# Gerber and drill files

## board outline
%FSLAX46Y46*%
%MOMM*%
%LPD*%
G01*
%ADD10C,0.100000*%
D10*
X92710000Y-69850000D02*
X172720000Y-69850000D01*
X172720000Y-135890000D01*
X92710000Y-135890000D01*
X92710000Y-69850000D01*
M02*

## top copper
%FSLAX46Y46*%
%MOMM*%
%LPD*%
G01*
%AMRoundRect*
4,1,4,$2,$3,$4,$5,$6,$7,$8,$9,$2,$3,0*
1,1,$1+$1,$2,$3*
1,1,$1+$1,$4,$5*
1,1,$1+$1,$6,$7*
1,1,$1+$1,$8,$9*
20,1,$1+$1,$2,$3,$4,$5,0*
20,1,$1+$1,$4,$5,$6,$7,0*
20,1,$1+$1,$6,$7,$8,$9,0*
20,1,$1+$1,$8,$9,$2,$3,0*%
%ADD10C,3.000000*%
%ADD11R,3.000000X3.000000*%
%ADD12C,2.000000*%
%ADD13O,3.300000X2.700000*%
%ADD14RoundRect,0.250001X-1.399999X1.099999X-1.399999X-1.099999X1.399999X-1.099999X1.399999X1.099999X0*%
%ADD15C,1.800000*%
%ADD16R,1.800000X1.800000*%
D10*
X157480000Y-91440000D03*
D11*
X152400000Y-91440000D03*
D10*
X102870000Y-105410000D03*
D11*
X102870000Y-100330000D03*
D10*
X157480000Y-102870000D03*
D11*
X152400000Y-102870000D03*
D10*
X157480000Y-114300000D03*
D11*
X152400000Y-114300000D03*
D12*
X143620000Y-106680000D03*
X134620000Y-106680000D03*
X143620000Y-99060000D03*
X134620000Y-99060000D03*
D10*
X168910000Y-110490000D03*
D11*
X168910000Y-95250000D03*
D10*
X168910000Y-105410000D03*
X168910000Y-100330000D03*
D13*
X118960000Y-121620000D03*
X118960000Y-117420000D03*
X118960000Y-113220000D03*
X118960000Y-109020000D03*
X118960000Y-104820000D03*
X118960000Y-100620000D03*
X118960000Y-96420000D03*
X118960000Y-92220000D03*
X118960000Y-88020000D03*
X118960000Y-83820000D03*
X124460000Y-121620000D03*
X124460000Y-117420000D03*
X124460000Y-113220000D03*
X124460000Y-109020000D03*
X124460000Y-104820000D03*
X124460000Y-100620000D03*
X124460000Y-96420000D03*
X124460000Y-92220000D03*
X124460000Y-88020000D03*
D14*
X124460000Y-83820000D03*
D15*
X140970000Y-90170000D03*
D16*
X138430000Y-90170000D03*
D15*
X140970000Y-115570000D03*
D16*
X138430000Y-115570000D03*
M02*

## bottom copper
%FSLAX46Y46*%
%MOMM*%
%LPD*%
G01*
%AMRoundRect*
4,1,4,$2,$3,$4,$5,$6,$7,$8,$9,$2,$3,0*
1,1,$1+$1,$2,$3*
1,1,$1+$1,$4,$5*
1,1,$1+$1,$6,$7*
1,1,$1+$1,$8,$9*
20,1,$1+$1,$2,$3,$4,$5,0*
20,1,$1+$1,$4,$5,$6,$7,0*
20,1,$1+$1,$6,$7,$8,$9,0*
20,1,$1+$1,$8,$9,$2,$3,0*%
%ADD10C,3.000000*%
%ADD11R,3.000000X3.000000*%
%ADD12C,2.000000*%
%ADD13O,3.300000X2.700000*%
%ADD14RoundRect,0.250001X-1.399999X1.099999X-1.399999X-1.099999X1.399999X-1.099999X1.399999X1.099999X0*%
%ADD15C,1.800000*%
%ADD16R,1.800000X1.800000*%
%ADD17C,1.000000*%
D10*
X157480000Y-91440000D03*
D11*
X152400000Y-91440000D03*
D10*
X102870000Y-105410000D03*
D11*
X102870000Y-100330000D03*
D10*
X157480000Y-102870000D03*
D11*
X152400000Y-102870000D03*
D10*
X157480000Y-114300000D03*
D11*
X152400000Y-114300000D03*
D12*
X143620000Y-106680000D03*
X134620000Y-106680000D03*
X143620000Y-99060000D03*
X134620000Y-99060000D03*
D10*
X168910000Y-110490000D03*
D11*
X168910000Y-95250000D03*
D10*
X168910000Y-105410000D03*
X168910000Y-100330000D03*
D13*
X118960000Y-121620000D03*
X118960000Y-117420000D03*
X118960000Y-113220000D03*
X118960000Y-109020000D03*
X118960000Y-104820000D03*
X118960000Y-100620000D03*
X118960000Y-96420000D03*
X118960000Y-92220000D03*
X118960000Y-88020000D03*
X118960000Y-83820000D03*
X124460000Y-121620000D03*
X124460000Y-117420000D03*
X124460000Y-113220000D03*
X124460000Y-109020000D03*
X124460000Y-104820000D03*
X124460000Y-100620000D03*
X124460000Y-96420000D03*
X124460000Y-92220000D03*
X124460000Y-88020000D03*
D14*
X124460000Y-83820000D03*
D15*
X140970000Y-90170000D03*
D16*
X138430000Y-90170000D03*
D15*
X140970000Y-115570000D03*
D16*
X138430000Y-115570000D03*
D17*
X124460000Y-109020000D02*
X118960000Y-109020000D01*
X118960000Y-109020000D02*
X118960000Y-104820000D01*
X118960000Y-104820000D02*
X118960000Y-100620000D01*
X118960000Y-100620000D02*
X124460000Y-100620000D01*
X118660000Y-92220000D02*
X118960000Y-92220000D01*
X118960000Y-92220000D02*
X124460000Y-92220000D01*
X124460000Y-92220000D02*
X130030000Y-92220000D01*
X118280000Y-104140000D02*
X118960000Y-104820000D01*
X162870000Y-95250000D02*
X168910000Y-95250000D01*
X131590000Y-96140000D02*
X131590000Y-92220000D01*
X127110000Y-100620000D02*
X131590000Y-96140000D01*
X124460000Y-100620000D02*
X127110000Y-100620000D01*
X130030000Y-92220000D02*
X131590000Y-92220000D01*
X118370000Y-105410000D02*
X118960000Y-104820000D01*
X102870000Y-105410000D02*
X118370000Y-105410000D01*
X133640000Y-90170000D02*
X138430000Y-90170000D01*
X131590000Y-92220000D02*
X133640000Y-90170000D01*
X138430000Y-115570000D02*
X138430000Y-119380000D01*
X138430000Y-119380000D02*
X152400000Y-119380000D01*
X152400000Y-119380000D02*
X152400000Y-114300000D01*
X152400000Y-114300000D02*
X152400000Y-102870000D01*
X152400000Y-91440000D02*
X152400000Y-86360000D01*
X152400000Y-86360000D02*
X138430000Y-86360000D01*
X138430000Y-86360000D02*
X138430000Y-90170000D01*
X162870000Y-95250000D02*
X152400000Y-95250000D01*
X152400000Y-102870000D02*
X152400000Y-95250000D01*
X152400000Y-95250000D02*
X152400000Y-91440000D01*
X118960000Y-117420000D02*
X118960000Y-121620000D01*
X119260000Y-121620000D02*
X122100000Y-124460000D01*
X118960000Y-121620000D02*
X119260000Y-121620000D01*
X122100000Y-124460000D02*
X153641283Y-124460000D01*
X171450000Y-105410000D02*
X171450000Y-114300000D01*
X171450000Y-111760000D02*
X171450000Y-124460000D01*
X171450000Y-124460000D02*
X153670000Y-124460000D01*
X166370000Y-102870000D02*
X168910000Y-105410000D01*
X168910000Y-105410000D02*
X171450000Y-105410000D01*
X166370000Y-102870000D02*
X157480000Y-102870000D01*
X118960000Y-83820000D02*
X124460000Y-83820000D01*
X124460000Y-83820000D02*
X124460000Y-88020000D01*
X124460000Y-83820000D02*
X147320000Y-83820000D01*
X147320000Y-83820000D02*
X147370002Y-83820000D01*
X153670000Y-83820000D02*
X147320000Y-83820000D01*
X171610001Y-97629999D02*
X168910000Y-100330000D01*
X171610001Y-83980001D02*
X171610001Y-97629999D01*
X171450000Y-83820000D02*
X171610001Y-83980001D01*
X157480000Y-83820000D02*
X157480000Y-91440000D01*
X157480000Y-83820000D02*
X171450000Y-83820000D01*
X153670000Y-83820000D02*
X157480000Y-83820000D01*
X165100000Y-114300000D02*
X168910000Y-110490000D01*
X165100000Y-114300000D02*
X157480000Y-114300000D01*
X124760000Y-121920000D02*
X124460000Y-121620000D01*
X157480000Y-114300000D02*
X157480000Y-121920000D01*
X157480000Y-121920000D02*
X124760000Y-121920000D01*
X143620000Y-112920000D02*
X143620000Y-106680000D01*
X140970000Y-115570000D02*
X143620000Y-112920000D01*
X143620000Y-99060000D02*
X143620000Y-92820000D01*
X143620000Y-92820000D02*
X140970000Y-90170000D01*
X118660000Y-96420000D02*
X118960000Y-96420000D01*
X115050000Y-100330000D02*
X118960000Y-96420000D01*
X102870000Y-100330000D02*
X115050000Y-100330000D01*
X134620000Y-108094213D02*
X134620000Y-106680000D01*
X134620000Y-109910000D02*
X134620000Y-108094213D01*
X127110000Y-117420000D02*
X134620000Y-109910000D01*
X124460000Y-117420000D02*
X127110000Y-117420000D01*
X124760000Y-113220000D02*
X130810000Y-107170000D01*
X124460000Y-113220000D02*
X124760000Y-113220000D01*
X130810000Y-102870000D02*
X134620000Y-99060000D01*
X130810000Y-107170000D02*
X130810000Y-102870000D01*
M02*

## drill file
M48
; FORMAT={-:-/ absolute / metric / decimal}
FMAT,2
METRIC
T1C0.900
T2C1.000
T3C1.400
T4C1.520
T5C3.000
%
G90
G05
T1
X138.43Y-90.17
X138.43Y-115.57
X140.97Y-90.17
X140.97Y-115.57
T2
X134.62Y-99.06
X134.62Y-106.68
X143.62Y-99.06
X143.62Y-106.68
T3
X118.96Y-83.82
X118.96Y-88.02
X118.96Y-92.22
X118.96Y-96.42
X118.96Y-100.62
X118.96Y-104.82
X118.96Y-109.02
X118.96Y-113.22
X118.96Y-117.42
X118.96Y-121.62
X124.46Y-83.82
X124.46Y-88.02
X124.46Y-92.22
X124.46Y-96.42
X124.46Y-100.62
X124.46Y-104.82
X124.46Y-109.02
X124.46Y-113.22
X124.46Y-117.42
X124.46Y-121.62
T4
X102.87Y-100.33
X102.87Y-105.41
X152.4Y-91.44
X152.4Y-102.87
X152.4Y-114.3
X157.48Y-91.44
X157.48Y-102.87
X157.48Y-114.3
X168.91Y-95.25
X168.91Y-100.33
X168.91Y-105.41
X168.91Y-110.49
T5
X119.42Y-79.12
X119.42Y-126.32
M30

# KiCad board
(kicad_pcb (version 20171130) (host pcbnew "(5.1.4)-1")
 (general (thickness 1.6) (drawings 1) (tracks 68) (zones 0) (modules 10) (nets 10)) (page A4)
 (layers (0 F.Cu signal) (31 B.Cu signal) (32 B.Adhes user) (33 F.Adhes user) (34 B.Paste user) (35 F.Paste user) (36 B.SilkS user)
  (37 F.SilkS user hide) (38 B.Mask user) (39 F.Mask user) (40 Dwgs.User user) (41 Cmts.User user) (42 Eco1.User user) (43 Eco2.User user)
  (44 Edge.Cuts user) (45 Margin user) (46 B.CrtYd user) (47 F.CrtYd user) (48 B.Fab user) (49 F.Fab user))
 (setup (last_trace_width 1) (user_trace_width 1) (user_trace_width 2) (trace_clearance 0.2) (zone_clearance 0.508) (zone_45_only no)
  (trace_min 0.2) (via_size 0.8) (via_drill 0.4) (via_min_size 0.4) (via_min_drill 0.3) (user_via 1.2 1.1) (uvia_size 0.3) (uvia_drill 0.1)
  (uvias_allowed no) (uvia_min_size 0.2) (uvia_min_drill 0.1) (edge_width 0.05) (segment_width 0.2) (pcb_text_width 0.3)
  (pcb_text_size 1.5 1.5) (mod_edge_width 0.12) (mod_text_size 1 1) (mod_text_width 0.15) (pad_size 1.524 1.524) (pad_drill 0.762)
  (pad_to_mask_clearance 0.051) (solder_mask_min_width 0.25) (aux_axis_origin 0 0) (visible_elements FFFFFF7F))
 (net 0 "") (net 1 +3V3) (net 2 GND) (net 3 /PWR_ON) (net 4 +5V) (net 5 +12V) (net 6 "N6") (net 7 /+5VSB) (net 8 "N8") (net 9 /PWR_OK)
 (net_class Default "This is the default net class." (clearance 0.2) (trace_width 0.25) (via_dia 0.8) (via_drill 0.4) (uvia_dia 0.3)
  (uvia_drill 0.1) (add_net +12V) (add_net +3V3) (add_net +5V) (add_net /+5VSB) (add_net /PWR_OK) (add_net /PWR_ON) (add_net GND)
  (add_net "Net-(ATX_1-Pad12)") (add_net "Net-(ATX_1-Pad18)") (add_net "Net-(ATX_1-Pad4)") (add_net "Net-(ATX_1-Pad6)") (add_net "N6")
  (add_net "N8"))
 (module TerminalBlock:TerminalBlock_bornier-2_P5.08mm (layer F.Cu) (at 152.4 91.44)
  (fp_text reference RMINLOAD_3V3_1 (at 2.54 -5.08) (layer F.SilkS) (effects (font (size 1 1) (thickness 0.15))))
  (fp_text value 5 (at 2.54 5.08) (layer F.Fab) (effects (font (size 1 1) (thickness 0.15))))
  (pad 2 thru_hole circle (at 5.08 0) (size 3 3) (drill 1.52) (layers *.Cu *.Mask) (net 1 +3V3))
  (pad 1 thru_hole rect (at 0 0) (size 3 3) (drill 1.52) (layers *.Cu *.Mask) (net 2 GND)))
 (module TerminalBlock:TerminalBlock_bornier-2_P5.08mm (layer F.Cu) (at 102.87 100.33 270)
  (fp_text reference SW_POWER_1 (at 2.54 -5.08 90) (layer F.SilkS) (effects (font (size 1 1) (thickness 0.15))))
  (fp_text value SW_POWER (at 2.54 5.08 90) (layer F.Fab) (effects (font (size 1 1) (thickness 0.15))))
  (pad 2 thru_hole circle (at 5.08 0 270) (size 3 3) (drill 1.52) (layers *.Cu *.Mask) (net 2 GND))
  (pad 1 thru_hole rect (at 0 0 270) (size 3 3) (drill 1.52) (layers *.Cu *.Mask) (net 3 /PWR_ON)))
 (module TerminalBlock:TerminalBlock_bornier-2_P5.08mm (layer F.Cu) (at 152.4 102.87)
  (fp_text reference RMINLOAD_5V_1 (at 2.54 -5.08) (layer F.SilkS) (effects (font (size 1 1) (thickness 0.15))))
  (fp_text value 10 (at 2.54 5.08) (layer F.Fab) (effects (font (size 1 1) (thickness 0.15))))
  (pad 2 thru_hole circle (at 5.08 0) (size 3 3) (drill 1.52) (layers *.Cu *.Mask) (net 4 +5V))
  (pad 1 thru_hole rect (at 0 0) (size 3 3) (drill 1.52) (layers *.Cu *.Mask) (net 2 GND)))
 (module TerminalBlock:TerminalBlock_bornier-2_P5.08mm (layer F.Cu) (at 152.4 114.3)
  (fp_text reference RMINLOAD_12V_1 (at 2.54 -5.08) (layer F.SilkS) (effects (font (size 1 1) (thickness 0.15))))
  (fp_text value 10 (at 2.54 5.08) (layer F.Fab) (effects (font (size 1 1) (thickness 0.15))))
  (pad 2 thru_hole circle (at 5.08 0) (size 3 3) (drill 1.52) (layers *.Cu *.Mask) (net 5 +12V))
  (pad 1 thru_hole rect (at 0 0) (size 3 3) (drill 1.52) (layers *.Cu *.Mask) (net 2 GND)))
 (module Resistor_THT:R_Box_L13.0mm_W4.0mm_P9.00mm (layer F.Cu) (at 134.62 106.68)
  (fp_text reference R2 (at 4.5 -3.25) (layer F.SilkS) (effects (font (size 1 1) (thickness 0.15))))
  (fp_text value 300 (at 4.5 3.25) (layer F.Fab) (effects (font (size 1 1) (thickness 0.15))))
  (pad 2 thru_hole circle (at 9 0) (size 2 2) (drill 1) (layers *.Cu *.Mask) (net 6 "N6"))
  (pad 1 thru_hole circle (at 0 0) (size 2 2) (drill 1) (layers *.Cu *.Mask) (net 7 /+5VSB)))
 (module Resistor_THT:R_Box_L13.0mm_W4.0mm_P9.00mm (layer F.Cu) (at 134.62 99.06)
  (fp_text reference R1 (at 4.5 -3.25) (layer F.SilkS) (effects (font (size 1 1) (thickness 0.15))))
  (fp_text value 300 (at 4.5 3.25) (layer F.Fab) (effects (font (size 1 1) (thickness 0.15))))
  (pad 2 thru_hole circle (at 9 0) (size 2 2) (drill 1) (layers *.Cu *.Mask) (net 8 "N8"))
  (pad 1 thru_hole circle (at 0 0) (size 2 2) (drill 1) (layers *.Cu *.Mask) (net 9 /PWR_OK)))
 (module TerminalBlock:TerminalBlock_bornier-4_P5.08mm (layer F.Cu) (at 168.91 95.25 270)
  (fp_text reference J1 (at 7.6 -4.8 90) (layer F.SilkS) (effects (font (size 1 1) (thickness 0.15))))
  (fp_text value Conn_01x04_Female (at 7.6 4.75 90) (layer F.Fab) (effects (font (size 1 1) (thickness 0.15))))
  (pad 4 thru_hole circle (at 15.24 0 270) (size 3 3) (drill 1.52) (layers *.Cu *.Mask) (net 5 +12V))
  (pad 1 thru_hole rect (at 0 0 270) (size 3 3) (drill 1.52) (layers *.Cu *.Mask) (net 2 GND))
  (pad 3 thru_hole circle (at 10.16 0 270) (size 3 3) (drill 1.52) (layers *.Cu *.Mask) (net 4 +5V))
  (pad 2 thru_hole circle (at 5.08 0 270) (size 3 3) (drill 1.52) (layers *.Cu *.Mask) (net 1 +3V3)))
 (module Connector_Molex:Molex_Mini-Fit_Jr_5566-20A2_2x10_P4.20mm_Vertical (layer F.Cu) (at 124.46 83.82 270)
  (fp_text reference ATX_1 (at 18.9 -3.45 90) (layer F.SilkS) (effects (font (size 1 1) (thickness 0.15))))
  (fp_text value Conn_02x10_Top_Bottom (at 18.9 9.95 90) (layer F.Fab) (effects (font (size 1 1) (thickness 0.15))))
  (pad "" np_thru_hole circle (at 42.5 5.04 270) (size 3 3) (drill 3) (layers *.Cu *.Mask))
  (pad "" np_thru_hole circle (at -4.7 5.04 270) (size 3 3) (drill 3) (layers *.Cu *.Mask))
  (pad 20 thru_hole oval (at 37.8 5.5 270) (size 2.7 3.3) (drill 1.4) (layers *.Cu *.Mask) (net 4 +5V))
  (pad 19 thru_hole oval (at 33.6 5.5 270) (size 2.7 3.3) (drill 1.4) (layers *.Cu *.Mask) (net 4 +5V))
  (pad 18 thru_hole oval (at 29.4 5.5 270) (size 2.7 3.3) (drill 1.4) (layers *.Cu *.Mask))
  (pad 17 thru_hole oval (at 25.2 5.5 270) (size 2.7 3.3) (drill 1.4) (layers *.Cu *.Mask) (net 2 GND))
  (pad 16 thru_hole oval (at 21 5.5 270) (size 2.7 3.3) (drill 1.4) (layers *.Cu *.Mask) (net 2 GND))
  (pad 15 thru_hole oval (at 16.8 5.5 270) (size 2.7 3.3) (drill 1.4) (layers *.Cu *.Mask) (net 2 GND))
  (pad 14 thru_hole oval (at 12.6 5.5 270) (size 2.7 3.3) (drill 1.4) (layers *.Cu *.Mask) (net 3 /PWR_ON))
  (pad 13 thru_hole oval (at 8.4 5.5 270) (size 2.7 3.3) (drill 1.4) (layers *.Cu *.Mask) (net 2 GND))
  (pad 12 thru_hole oval (at 4.2 5.5 270) (size 2.7 3.3) (drill 1.4) (layers *.Cu *.Mask))
  (pad 11 thru_hole oval (at 0 5.5 270) (size 2.7 3.3) (drill 1.4) (layers *.Cu *.Mask) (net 1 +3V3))
  (pad 10 thru_hole oval (at 37.8 0 270) (size 2.7 3.3) (drill 1.4) (layers *.Cu *.Mask) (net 5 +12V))
  (pad 9 thru_hole oval (at 33.6 0 270) (size 2.7 3.3) (drill 1.4) (layers *.Cu *.Mask) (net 7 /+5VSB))
  (pad 8 thru_hole oval (at 29.4 0 270) (size 2.7 3.3) (drill 1.4) (layers *.Cu *.Mask) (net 9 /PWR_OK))
  (pad 7 thru_hole oval (at 25.2 0 270) (size 2.7 3.3) (drill 1.4) (layers *.Cu *.Mask) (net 2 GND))
  (pad 6 thru_hole oval (at 21 0 270) (size 2.7 3.3) (drill 1.4) (layers *.Cu *.Mask))
  (pad 5 thru_hole oval (at 16.8 0 270) (size 2.7 3.3) (drill 1.4) (layers *.Cu *.Mask) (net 2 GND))
  (pad 4 thru_hole oval (at 12.6 0 270) (size 2.7 3.3) (drill 1.4) (layers *.Cu *.Mask))
  (pad 3 thru_hole oval (at 8.4 0 270) (size 2.7 3.3) (drill 1.4) (layers *.Cu *.Mask) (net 2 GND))
  (pad 2 thru_hole oval (at 4.2 0 270) (size 2.7 3.3) (drill 1.4) (layers *.Cu *.Mask) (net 1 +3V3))
  (pad 1 thru_hole roundrect (at 0 0 270) (size 2.7 3.3) (drill 1.4) (layers *.Cu *.Mask) (roundrect_rratio 0.09259299999999999)
   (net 1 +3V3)))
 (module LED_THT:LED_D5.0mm (layer F.Cu) (at 138.43 90.17)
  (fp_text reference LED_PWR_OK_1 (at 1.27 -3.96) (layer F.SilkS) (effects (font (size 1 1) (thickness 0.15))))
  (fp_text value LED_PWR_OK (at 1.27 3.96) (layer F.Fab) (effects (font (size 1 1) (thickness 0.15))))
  (pad 2 thru_hole circle (at 2.54 0) (size 1.8 1.8) (drill 0.9) (layers *.Cu *.Mask) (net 8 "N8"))
  (pad 1 thru_hole rect (at 0 0) (size 1.8 1.8) (drill 0.9) (layers *.Cu *.Mask) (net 2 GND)))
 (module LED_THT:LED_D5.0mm (layer F.Cu) (at 138.43 115.57)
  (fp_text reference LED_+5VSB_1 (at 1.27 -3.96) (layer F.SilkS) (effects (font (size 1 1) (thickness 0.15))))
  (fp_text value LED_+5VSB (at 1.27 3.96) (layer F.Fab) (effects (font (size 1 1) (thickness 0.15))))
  (pad 2 thru_hole circle (at 2.54 0) (size 1.8 1.8) (drill 0.9) (layers *.Cu *.Mask) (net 6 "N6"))
  (pad 1 thru_hole rect (at 0 0) (size 1.8 1.8) (drill 0.9) (layers *.Cu *.Mask) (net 2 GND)))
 (gr_poly (pts (xy 92.71 69.85) (xy 172.72 69.85) (xy 172.72 135.89) (xy 92.71 135.89)) (layer Edge.Cuts) (width 0.1))
 (segment (start 124.46 109.02) (end 118.96 109.02) (width 1) (layer B.Cu) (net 2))
 (segment (start 118.96 109.02) (end 118.96 104.82) (width 1) (layer B.Cu) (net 2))
 (segment (start 118.96 104.82) (end 118.96 100.62) (width 1) (layer B.Cu) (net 2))
 (segment (start 118.96 100.62) (end 124.46 100.62) (width 1) (layer B.Cu) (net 2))
 (segment (start 118.66 92.22) (end 118.96 92.22) (width 1) (layer B.Cu) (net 2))
 (segment (start 118.96 92.22) (end 124.46 92.22) (width 1) (layer B.Cu) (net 2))
 (segment (start 124.46 92.22) (end 130.03 92.22) (width 1) (layer B.Cu) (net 2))
 (segment (start 118.28 104.14) (end 118.96 104.82) (width 1) (layer B.Cu) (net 2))
 (segment (start 162.87 95.25) (end 168.91 95.25) (width 1) (layer B.Cu) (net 2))
 (segment (start 131.59 96.14) (end 131.59 92.22) (width 1) (layer B.Cu) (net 2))
 (segment (start 127.11 100.62) (end 131.59 96.14) (width 1) (layer B.Cu) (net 2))
 (segment (start 124.46 100.62) (end 127.11 100.62) (width 1) (layer B.Cu) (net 2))
 (segment (start 130.03 92.22) (end 131.59 92.22) (width 1) (layer B.Cu) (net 2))
 (segment (start 118.37 105.41) (end 118.96 104.82) (width 1) (layer B.Cu) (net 2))
 (segment (start 102.87 105.41) (end 118.37 105.41) (width 1) (layer B.Cu) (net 2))
 (segment (start 133.64 90.17) (end 138.43 90.17) (width 1) (layer B.Cu) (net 2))
 (segment (start 131.59 92.22) (end 133.64 90.17) (width 1) (layer B.Cu) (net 2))
 (segment (start 138.43 115.57) (end 138.43 119.38) (width 1) (layer B.Cu) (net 2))
 (segment (start 138.43 119.38) (end 152.4 119.38) (width 1) (layer B.Cu) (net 2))
 (segment (start 152.4 119.38) (end 152.4 114.3) (width 1) (layer B.Cu) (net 2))
 (segment (start 152.4 114.3) (end 152.4 102.87) (width 1) (layer B.Cu) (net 2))
 (segment (start 152.4 91.44) (end 152.4 86.36) (width 1) (layer B.Cu) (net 2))
 (segment (start 152.4 86.36) (end 138.43 86.36) (width 1) (layer B.Cu) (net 2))
 (segment (start 138.43 86.36) (end 138.43 90.17) (width 1) (layer B.Cu) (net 2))
 (segment (start 162.87 95.25) (end 152.4 95.25) (width 1) (layer B.Cu) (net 2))
 (segment (start 152.4 102.87) (end 152.4 95.25) (width 1) (layer B.Cu) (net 2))
 (segment (start 152.4 95.25) (end 152.4 91.44) (width 1) (layer B.Cu) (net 2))
 (segment (start 118.96 117.42) (end 118.96 121.62) (width 1) (layer B.Cu) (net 4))
 (segment (start 119.26 121.62) (end 122.1 124.46) (width 1) (layer B.Cu) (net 4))
 (segment (start 118.96 121.62) (end 119.26 121.62) (width 1) (layer B.Cu) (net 4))
 (segment (start 122.1 124.46) (end 153.641283 124.46) (width 1) (layer B.Cu) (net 4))
 (segment (start 171.45 105.41) (end 171.45 114.3) (width 1) (layer B.Cu) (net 4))
 (segment (start 171.45 111.76) (end 171.45 124.46) (width 1) (layer B.Cu) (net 4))
 (segment (start 171.45 124.46) (end 153.67 124.46) (width 1) (layer B.Cu) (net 4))
 (segment (start 166.37 102.87) (end 168.91 105.41) (width 1) (layer B.Cu) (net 4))
 (segment (start 168.91 105.41) (end 171.45 105.41) (width 1) (layer B.Cu) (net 4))
 (segment (start 166.37 102.87) (end 157.48 102.87) (width 1) (layer B.Cu) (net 4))
 (segment (start 118.96 83.82) (end 124.46 83.82) (width 1) (layer B.Cu) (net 1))
 (segment (start 124.46 83.82) (end 124.46 88.02) (width 1) (layer B.Cu) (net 1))
 (segment (start 124.46 83.82) (end 147.32 83.82) (width 1) (layer B.Cu) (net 1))
 (segment (start 147.32 83.82) (end 147.370002 83.82) (width 1) (layer B.Cu) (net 1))
 (segment (start 153.67 83.82) (end 147.32 83.82) (width 1) (layer B.Cu) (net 1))
 (segment (start 171.610001 97.629999) (end 168.91 100.33) (width 1) (layer B.Cu) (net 1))
 (segment (start 171.610001 83.980001) (end 171.610001 97.629999) (width 1) (layer B.Cu) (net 1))
 (segment (start 171.45 83.82) (end 171.610001 83.980001) (width 1) (layer B.Cu) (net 1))
 (segment (start 157.48 83.82) (end 157.48 91.44) (width 1) (layer B.Cu) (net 1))
 (segment (start 157.48 83.82) (end 171.45 83.82) (width 1) (layer B.Cu) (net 1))
 (segment (start 153.67 83.82) (end 157.48 83.82) (width 1) (layer B.Cu) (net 1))
 (segment (start 165.1 114.3) (end 168.91 110.49) (width 1) (layer B.Cu) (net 5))
 (segment (start 165.1 114.3) (end 157.48 114.3) (width 1) (layer B.Cu) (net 5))
 (segment (start 124.76 121.92) (end 124.46 121.62) (width 1) (layer B.Cu) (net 5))
 (segment (start 157.48 114.3) (end 157.48 121.92) (width 1) (layer B.Cu) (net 5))
 (segment (start 157.48 121.92) (end 124.76 121.92) (width 1) (layer B.Cu) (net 5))
 (segment (start 143.62 112.92) (end 143.62 106.68) (width 1) (layer B.Cu) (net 6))
 (segment (start 140.97 115.57) (end 143.62 112.92) (width 1) (layer B.Cu) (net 6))
 (segment (start 143.62 99.06) (end 143.62 92.82) (width 1) (layer B.Cu) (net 8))
 (segment (start 143.62 92.82) (end 140.97 90.17) (width 1) (layer B.Cu) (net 8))
 (segment (start 118.66 96.42) (end 118.96 96.42) (width 1) (layer B.Cu) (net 3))
 (segment (start 115.05 100.33) (end 118.96 96.42) (width 1) (layer B.Cu) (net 3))
 (segment (start 102.87 100.33) (end 115.05 100.33) (width 1) (layer B.Cu) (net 3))
 (segment (start 134.62 108.094213) (end 134.62 106.68) (width 1) (layer B.Cu) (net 7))
 (segment (start 134.62 109.91) (end 134.62 108.094213) (width 1) (layer B.Cu) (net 7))
 (segment (start 127.11 117.42) (end 134.62 109.91) (width 1) (layer B.Cu) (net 7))
 (segment (start 124.46 117.42) (end 127.11 117.42) (width 1) (layer B.Cu) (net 7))
 (segment (start 124.76 113.22) (end 130.81 107.17) (width 1) (layer B.Cu) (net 9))
 (segment (start 124.46 113.22) (end 124.76 113.22) (width 1) (layer B.Cu) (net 9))
 (segment (start 130.81 102.87) (end 134.62 99.06) (width 1) (layer B.Cu) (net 9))
 (segment (start 130.81 107.17) (end 130.81 102.87) (width 1) (layer B.Cu) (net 9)))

